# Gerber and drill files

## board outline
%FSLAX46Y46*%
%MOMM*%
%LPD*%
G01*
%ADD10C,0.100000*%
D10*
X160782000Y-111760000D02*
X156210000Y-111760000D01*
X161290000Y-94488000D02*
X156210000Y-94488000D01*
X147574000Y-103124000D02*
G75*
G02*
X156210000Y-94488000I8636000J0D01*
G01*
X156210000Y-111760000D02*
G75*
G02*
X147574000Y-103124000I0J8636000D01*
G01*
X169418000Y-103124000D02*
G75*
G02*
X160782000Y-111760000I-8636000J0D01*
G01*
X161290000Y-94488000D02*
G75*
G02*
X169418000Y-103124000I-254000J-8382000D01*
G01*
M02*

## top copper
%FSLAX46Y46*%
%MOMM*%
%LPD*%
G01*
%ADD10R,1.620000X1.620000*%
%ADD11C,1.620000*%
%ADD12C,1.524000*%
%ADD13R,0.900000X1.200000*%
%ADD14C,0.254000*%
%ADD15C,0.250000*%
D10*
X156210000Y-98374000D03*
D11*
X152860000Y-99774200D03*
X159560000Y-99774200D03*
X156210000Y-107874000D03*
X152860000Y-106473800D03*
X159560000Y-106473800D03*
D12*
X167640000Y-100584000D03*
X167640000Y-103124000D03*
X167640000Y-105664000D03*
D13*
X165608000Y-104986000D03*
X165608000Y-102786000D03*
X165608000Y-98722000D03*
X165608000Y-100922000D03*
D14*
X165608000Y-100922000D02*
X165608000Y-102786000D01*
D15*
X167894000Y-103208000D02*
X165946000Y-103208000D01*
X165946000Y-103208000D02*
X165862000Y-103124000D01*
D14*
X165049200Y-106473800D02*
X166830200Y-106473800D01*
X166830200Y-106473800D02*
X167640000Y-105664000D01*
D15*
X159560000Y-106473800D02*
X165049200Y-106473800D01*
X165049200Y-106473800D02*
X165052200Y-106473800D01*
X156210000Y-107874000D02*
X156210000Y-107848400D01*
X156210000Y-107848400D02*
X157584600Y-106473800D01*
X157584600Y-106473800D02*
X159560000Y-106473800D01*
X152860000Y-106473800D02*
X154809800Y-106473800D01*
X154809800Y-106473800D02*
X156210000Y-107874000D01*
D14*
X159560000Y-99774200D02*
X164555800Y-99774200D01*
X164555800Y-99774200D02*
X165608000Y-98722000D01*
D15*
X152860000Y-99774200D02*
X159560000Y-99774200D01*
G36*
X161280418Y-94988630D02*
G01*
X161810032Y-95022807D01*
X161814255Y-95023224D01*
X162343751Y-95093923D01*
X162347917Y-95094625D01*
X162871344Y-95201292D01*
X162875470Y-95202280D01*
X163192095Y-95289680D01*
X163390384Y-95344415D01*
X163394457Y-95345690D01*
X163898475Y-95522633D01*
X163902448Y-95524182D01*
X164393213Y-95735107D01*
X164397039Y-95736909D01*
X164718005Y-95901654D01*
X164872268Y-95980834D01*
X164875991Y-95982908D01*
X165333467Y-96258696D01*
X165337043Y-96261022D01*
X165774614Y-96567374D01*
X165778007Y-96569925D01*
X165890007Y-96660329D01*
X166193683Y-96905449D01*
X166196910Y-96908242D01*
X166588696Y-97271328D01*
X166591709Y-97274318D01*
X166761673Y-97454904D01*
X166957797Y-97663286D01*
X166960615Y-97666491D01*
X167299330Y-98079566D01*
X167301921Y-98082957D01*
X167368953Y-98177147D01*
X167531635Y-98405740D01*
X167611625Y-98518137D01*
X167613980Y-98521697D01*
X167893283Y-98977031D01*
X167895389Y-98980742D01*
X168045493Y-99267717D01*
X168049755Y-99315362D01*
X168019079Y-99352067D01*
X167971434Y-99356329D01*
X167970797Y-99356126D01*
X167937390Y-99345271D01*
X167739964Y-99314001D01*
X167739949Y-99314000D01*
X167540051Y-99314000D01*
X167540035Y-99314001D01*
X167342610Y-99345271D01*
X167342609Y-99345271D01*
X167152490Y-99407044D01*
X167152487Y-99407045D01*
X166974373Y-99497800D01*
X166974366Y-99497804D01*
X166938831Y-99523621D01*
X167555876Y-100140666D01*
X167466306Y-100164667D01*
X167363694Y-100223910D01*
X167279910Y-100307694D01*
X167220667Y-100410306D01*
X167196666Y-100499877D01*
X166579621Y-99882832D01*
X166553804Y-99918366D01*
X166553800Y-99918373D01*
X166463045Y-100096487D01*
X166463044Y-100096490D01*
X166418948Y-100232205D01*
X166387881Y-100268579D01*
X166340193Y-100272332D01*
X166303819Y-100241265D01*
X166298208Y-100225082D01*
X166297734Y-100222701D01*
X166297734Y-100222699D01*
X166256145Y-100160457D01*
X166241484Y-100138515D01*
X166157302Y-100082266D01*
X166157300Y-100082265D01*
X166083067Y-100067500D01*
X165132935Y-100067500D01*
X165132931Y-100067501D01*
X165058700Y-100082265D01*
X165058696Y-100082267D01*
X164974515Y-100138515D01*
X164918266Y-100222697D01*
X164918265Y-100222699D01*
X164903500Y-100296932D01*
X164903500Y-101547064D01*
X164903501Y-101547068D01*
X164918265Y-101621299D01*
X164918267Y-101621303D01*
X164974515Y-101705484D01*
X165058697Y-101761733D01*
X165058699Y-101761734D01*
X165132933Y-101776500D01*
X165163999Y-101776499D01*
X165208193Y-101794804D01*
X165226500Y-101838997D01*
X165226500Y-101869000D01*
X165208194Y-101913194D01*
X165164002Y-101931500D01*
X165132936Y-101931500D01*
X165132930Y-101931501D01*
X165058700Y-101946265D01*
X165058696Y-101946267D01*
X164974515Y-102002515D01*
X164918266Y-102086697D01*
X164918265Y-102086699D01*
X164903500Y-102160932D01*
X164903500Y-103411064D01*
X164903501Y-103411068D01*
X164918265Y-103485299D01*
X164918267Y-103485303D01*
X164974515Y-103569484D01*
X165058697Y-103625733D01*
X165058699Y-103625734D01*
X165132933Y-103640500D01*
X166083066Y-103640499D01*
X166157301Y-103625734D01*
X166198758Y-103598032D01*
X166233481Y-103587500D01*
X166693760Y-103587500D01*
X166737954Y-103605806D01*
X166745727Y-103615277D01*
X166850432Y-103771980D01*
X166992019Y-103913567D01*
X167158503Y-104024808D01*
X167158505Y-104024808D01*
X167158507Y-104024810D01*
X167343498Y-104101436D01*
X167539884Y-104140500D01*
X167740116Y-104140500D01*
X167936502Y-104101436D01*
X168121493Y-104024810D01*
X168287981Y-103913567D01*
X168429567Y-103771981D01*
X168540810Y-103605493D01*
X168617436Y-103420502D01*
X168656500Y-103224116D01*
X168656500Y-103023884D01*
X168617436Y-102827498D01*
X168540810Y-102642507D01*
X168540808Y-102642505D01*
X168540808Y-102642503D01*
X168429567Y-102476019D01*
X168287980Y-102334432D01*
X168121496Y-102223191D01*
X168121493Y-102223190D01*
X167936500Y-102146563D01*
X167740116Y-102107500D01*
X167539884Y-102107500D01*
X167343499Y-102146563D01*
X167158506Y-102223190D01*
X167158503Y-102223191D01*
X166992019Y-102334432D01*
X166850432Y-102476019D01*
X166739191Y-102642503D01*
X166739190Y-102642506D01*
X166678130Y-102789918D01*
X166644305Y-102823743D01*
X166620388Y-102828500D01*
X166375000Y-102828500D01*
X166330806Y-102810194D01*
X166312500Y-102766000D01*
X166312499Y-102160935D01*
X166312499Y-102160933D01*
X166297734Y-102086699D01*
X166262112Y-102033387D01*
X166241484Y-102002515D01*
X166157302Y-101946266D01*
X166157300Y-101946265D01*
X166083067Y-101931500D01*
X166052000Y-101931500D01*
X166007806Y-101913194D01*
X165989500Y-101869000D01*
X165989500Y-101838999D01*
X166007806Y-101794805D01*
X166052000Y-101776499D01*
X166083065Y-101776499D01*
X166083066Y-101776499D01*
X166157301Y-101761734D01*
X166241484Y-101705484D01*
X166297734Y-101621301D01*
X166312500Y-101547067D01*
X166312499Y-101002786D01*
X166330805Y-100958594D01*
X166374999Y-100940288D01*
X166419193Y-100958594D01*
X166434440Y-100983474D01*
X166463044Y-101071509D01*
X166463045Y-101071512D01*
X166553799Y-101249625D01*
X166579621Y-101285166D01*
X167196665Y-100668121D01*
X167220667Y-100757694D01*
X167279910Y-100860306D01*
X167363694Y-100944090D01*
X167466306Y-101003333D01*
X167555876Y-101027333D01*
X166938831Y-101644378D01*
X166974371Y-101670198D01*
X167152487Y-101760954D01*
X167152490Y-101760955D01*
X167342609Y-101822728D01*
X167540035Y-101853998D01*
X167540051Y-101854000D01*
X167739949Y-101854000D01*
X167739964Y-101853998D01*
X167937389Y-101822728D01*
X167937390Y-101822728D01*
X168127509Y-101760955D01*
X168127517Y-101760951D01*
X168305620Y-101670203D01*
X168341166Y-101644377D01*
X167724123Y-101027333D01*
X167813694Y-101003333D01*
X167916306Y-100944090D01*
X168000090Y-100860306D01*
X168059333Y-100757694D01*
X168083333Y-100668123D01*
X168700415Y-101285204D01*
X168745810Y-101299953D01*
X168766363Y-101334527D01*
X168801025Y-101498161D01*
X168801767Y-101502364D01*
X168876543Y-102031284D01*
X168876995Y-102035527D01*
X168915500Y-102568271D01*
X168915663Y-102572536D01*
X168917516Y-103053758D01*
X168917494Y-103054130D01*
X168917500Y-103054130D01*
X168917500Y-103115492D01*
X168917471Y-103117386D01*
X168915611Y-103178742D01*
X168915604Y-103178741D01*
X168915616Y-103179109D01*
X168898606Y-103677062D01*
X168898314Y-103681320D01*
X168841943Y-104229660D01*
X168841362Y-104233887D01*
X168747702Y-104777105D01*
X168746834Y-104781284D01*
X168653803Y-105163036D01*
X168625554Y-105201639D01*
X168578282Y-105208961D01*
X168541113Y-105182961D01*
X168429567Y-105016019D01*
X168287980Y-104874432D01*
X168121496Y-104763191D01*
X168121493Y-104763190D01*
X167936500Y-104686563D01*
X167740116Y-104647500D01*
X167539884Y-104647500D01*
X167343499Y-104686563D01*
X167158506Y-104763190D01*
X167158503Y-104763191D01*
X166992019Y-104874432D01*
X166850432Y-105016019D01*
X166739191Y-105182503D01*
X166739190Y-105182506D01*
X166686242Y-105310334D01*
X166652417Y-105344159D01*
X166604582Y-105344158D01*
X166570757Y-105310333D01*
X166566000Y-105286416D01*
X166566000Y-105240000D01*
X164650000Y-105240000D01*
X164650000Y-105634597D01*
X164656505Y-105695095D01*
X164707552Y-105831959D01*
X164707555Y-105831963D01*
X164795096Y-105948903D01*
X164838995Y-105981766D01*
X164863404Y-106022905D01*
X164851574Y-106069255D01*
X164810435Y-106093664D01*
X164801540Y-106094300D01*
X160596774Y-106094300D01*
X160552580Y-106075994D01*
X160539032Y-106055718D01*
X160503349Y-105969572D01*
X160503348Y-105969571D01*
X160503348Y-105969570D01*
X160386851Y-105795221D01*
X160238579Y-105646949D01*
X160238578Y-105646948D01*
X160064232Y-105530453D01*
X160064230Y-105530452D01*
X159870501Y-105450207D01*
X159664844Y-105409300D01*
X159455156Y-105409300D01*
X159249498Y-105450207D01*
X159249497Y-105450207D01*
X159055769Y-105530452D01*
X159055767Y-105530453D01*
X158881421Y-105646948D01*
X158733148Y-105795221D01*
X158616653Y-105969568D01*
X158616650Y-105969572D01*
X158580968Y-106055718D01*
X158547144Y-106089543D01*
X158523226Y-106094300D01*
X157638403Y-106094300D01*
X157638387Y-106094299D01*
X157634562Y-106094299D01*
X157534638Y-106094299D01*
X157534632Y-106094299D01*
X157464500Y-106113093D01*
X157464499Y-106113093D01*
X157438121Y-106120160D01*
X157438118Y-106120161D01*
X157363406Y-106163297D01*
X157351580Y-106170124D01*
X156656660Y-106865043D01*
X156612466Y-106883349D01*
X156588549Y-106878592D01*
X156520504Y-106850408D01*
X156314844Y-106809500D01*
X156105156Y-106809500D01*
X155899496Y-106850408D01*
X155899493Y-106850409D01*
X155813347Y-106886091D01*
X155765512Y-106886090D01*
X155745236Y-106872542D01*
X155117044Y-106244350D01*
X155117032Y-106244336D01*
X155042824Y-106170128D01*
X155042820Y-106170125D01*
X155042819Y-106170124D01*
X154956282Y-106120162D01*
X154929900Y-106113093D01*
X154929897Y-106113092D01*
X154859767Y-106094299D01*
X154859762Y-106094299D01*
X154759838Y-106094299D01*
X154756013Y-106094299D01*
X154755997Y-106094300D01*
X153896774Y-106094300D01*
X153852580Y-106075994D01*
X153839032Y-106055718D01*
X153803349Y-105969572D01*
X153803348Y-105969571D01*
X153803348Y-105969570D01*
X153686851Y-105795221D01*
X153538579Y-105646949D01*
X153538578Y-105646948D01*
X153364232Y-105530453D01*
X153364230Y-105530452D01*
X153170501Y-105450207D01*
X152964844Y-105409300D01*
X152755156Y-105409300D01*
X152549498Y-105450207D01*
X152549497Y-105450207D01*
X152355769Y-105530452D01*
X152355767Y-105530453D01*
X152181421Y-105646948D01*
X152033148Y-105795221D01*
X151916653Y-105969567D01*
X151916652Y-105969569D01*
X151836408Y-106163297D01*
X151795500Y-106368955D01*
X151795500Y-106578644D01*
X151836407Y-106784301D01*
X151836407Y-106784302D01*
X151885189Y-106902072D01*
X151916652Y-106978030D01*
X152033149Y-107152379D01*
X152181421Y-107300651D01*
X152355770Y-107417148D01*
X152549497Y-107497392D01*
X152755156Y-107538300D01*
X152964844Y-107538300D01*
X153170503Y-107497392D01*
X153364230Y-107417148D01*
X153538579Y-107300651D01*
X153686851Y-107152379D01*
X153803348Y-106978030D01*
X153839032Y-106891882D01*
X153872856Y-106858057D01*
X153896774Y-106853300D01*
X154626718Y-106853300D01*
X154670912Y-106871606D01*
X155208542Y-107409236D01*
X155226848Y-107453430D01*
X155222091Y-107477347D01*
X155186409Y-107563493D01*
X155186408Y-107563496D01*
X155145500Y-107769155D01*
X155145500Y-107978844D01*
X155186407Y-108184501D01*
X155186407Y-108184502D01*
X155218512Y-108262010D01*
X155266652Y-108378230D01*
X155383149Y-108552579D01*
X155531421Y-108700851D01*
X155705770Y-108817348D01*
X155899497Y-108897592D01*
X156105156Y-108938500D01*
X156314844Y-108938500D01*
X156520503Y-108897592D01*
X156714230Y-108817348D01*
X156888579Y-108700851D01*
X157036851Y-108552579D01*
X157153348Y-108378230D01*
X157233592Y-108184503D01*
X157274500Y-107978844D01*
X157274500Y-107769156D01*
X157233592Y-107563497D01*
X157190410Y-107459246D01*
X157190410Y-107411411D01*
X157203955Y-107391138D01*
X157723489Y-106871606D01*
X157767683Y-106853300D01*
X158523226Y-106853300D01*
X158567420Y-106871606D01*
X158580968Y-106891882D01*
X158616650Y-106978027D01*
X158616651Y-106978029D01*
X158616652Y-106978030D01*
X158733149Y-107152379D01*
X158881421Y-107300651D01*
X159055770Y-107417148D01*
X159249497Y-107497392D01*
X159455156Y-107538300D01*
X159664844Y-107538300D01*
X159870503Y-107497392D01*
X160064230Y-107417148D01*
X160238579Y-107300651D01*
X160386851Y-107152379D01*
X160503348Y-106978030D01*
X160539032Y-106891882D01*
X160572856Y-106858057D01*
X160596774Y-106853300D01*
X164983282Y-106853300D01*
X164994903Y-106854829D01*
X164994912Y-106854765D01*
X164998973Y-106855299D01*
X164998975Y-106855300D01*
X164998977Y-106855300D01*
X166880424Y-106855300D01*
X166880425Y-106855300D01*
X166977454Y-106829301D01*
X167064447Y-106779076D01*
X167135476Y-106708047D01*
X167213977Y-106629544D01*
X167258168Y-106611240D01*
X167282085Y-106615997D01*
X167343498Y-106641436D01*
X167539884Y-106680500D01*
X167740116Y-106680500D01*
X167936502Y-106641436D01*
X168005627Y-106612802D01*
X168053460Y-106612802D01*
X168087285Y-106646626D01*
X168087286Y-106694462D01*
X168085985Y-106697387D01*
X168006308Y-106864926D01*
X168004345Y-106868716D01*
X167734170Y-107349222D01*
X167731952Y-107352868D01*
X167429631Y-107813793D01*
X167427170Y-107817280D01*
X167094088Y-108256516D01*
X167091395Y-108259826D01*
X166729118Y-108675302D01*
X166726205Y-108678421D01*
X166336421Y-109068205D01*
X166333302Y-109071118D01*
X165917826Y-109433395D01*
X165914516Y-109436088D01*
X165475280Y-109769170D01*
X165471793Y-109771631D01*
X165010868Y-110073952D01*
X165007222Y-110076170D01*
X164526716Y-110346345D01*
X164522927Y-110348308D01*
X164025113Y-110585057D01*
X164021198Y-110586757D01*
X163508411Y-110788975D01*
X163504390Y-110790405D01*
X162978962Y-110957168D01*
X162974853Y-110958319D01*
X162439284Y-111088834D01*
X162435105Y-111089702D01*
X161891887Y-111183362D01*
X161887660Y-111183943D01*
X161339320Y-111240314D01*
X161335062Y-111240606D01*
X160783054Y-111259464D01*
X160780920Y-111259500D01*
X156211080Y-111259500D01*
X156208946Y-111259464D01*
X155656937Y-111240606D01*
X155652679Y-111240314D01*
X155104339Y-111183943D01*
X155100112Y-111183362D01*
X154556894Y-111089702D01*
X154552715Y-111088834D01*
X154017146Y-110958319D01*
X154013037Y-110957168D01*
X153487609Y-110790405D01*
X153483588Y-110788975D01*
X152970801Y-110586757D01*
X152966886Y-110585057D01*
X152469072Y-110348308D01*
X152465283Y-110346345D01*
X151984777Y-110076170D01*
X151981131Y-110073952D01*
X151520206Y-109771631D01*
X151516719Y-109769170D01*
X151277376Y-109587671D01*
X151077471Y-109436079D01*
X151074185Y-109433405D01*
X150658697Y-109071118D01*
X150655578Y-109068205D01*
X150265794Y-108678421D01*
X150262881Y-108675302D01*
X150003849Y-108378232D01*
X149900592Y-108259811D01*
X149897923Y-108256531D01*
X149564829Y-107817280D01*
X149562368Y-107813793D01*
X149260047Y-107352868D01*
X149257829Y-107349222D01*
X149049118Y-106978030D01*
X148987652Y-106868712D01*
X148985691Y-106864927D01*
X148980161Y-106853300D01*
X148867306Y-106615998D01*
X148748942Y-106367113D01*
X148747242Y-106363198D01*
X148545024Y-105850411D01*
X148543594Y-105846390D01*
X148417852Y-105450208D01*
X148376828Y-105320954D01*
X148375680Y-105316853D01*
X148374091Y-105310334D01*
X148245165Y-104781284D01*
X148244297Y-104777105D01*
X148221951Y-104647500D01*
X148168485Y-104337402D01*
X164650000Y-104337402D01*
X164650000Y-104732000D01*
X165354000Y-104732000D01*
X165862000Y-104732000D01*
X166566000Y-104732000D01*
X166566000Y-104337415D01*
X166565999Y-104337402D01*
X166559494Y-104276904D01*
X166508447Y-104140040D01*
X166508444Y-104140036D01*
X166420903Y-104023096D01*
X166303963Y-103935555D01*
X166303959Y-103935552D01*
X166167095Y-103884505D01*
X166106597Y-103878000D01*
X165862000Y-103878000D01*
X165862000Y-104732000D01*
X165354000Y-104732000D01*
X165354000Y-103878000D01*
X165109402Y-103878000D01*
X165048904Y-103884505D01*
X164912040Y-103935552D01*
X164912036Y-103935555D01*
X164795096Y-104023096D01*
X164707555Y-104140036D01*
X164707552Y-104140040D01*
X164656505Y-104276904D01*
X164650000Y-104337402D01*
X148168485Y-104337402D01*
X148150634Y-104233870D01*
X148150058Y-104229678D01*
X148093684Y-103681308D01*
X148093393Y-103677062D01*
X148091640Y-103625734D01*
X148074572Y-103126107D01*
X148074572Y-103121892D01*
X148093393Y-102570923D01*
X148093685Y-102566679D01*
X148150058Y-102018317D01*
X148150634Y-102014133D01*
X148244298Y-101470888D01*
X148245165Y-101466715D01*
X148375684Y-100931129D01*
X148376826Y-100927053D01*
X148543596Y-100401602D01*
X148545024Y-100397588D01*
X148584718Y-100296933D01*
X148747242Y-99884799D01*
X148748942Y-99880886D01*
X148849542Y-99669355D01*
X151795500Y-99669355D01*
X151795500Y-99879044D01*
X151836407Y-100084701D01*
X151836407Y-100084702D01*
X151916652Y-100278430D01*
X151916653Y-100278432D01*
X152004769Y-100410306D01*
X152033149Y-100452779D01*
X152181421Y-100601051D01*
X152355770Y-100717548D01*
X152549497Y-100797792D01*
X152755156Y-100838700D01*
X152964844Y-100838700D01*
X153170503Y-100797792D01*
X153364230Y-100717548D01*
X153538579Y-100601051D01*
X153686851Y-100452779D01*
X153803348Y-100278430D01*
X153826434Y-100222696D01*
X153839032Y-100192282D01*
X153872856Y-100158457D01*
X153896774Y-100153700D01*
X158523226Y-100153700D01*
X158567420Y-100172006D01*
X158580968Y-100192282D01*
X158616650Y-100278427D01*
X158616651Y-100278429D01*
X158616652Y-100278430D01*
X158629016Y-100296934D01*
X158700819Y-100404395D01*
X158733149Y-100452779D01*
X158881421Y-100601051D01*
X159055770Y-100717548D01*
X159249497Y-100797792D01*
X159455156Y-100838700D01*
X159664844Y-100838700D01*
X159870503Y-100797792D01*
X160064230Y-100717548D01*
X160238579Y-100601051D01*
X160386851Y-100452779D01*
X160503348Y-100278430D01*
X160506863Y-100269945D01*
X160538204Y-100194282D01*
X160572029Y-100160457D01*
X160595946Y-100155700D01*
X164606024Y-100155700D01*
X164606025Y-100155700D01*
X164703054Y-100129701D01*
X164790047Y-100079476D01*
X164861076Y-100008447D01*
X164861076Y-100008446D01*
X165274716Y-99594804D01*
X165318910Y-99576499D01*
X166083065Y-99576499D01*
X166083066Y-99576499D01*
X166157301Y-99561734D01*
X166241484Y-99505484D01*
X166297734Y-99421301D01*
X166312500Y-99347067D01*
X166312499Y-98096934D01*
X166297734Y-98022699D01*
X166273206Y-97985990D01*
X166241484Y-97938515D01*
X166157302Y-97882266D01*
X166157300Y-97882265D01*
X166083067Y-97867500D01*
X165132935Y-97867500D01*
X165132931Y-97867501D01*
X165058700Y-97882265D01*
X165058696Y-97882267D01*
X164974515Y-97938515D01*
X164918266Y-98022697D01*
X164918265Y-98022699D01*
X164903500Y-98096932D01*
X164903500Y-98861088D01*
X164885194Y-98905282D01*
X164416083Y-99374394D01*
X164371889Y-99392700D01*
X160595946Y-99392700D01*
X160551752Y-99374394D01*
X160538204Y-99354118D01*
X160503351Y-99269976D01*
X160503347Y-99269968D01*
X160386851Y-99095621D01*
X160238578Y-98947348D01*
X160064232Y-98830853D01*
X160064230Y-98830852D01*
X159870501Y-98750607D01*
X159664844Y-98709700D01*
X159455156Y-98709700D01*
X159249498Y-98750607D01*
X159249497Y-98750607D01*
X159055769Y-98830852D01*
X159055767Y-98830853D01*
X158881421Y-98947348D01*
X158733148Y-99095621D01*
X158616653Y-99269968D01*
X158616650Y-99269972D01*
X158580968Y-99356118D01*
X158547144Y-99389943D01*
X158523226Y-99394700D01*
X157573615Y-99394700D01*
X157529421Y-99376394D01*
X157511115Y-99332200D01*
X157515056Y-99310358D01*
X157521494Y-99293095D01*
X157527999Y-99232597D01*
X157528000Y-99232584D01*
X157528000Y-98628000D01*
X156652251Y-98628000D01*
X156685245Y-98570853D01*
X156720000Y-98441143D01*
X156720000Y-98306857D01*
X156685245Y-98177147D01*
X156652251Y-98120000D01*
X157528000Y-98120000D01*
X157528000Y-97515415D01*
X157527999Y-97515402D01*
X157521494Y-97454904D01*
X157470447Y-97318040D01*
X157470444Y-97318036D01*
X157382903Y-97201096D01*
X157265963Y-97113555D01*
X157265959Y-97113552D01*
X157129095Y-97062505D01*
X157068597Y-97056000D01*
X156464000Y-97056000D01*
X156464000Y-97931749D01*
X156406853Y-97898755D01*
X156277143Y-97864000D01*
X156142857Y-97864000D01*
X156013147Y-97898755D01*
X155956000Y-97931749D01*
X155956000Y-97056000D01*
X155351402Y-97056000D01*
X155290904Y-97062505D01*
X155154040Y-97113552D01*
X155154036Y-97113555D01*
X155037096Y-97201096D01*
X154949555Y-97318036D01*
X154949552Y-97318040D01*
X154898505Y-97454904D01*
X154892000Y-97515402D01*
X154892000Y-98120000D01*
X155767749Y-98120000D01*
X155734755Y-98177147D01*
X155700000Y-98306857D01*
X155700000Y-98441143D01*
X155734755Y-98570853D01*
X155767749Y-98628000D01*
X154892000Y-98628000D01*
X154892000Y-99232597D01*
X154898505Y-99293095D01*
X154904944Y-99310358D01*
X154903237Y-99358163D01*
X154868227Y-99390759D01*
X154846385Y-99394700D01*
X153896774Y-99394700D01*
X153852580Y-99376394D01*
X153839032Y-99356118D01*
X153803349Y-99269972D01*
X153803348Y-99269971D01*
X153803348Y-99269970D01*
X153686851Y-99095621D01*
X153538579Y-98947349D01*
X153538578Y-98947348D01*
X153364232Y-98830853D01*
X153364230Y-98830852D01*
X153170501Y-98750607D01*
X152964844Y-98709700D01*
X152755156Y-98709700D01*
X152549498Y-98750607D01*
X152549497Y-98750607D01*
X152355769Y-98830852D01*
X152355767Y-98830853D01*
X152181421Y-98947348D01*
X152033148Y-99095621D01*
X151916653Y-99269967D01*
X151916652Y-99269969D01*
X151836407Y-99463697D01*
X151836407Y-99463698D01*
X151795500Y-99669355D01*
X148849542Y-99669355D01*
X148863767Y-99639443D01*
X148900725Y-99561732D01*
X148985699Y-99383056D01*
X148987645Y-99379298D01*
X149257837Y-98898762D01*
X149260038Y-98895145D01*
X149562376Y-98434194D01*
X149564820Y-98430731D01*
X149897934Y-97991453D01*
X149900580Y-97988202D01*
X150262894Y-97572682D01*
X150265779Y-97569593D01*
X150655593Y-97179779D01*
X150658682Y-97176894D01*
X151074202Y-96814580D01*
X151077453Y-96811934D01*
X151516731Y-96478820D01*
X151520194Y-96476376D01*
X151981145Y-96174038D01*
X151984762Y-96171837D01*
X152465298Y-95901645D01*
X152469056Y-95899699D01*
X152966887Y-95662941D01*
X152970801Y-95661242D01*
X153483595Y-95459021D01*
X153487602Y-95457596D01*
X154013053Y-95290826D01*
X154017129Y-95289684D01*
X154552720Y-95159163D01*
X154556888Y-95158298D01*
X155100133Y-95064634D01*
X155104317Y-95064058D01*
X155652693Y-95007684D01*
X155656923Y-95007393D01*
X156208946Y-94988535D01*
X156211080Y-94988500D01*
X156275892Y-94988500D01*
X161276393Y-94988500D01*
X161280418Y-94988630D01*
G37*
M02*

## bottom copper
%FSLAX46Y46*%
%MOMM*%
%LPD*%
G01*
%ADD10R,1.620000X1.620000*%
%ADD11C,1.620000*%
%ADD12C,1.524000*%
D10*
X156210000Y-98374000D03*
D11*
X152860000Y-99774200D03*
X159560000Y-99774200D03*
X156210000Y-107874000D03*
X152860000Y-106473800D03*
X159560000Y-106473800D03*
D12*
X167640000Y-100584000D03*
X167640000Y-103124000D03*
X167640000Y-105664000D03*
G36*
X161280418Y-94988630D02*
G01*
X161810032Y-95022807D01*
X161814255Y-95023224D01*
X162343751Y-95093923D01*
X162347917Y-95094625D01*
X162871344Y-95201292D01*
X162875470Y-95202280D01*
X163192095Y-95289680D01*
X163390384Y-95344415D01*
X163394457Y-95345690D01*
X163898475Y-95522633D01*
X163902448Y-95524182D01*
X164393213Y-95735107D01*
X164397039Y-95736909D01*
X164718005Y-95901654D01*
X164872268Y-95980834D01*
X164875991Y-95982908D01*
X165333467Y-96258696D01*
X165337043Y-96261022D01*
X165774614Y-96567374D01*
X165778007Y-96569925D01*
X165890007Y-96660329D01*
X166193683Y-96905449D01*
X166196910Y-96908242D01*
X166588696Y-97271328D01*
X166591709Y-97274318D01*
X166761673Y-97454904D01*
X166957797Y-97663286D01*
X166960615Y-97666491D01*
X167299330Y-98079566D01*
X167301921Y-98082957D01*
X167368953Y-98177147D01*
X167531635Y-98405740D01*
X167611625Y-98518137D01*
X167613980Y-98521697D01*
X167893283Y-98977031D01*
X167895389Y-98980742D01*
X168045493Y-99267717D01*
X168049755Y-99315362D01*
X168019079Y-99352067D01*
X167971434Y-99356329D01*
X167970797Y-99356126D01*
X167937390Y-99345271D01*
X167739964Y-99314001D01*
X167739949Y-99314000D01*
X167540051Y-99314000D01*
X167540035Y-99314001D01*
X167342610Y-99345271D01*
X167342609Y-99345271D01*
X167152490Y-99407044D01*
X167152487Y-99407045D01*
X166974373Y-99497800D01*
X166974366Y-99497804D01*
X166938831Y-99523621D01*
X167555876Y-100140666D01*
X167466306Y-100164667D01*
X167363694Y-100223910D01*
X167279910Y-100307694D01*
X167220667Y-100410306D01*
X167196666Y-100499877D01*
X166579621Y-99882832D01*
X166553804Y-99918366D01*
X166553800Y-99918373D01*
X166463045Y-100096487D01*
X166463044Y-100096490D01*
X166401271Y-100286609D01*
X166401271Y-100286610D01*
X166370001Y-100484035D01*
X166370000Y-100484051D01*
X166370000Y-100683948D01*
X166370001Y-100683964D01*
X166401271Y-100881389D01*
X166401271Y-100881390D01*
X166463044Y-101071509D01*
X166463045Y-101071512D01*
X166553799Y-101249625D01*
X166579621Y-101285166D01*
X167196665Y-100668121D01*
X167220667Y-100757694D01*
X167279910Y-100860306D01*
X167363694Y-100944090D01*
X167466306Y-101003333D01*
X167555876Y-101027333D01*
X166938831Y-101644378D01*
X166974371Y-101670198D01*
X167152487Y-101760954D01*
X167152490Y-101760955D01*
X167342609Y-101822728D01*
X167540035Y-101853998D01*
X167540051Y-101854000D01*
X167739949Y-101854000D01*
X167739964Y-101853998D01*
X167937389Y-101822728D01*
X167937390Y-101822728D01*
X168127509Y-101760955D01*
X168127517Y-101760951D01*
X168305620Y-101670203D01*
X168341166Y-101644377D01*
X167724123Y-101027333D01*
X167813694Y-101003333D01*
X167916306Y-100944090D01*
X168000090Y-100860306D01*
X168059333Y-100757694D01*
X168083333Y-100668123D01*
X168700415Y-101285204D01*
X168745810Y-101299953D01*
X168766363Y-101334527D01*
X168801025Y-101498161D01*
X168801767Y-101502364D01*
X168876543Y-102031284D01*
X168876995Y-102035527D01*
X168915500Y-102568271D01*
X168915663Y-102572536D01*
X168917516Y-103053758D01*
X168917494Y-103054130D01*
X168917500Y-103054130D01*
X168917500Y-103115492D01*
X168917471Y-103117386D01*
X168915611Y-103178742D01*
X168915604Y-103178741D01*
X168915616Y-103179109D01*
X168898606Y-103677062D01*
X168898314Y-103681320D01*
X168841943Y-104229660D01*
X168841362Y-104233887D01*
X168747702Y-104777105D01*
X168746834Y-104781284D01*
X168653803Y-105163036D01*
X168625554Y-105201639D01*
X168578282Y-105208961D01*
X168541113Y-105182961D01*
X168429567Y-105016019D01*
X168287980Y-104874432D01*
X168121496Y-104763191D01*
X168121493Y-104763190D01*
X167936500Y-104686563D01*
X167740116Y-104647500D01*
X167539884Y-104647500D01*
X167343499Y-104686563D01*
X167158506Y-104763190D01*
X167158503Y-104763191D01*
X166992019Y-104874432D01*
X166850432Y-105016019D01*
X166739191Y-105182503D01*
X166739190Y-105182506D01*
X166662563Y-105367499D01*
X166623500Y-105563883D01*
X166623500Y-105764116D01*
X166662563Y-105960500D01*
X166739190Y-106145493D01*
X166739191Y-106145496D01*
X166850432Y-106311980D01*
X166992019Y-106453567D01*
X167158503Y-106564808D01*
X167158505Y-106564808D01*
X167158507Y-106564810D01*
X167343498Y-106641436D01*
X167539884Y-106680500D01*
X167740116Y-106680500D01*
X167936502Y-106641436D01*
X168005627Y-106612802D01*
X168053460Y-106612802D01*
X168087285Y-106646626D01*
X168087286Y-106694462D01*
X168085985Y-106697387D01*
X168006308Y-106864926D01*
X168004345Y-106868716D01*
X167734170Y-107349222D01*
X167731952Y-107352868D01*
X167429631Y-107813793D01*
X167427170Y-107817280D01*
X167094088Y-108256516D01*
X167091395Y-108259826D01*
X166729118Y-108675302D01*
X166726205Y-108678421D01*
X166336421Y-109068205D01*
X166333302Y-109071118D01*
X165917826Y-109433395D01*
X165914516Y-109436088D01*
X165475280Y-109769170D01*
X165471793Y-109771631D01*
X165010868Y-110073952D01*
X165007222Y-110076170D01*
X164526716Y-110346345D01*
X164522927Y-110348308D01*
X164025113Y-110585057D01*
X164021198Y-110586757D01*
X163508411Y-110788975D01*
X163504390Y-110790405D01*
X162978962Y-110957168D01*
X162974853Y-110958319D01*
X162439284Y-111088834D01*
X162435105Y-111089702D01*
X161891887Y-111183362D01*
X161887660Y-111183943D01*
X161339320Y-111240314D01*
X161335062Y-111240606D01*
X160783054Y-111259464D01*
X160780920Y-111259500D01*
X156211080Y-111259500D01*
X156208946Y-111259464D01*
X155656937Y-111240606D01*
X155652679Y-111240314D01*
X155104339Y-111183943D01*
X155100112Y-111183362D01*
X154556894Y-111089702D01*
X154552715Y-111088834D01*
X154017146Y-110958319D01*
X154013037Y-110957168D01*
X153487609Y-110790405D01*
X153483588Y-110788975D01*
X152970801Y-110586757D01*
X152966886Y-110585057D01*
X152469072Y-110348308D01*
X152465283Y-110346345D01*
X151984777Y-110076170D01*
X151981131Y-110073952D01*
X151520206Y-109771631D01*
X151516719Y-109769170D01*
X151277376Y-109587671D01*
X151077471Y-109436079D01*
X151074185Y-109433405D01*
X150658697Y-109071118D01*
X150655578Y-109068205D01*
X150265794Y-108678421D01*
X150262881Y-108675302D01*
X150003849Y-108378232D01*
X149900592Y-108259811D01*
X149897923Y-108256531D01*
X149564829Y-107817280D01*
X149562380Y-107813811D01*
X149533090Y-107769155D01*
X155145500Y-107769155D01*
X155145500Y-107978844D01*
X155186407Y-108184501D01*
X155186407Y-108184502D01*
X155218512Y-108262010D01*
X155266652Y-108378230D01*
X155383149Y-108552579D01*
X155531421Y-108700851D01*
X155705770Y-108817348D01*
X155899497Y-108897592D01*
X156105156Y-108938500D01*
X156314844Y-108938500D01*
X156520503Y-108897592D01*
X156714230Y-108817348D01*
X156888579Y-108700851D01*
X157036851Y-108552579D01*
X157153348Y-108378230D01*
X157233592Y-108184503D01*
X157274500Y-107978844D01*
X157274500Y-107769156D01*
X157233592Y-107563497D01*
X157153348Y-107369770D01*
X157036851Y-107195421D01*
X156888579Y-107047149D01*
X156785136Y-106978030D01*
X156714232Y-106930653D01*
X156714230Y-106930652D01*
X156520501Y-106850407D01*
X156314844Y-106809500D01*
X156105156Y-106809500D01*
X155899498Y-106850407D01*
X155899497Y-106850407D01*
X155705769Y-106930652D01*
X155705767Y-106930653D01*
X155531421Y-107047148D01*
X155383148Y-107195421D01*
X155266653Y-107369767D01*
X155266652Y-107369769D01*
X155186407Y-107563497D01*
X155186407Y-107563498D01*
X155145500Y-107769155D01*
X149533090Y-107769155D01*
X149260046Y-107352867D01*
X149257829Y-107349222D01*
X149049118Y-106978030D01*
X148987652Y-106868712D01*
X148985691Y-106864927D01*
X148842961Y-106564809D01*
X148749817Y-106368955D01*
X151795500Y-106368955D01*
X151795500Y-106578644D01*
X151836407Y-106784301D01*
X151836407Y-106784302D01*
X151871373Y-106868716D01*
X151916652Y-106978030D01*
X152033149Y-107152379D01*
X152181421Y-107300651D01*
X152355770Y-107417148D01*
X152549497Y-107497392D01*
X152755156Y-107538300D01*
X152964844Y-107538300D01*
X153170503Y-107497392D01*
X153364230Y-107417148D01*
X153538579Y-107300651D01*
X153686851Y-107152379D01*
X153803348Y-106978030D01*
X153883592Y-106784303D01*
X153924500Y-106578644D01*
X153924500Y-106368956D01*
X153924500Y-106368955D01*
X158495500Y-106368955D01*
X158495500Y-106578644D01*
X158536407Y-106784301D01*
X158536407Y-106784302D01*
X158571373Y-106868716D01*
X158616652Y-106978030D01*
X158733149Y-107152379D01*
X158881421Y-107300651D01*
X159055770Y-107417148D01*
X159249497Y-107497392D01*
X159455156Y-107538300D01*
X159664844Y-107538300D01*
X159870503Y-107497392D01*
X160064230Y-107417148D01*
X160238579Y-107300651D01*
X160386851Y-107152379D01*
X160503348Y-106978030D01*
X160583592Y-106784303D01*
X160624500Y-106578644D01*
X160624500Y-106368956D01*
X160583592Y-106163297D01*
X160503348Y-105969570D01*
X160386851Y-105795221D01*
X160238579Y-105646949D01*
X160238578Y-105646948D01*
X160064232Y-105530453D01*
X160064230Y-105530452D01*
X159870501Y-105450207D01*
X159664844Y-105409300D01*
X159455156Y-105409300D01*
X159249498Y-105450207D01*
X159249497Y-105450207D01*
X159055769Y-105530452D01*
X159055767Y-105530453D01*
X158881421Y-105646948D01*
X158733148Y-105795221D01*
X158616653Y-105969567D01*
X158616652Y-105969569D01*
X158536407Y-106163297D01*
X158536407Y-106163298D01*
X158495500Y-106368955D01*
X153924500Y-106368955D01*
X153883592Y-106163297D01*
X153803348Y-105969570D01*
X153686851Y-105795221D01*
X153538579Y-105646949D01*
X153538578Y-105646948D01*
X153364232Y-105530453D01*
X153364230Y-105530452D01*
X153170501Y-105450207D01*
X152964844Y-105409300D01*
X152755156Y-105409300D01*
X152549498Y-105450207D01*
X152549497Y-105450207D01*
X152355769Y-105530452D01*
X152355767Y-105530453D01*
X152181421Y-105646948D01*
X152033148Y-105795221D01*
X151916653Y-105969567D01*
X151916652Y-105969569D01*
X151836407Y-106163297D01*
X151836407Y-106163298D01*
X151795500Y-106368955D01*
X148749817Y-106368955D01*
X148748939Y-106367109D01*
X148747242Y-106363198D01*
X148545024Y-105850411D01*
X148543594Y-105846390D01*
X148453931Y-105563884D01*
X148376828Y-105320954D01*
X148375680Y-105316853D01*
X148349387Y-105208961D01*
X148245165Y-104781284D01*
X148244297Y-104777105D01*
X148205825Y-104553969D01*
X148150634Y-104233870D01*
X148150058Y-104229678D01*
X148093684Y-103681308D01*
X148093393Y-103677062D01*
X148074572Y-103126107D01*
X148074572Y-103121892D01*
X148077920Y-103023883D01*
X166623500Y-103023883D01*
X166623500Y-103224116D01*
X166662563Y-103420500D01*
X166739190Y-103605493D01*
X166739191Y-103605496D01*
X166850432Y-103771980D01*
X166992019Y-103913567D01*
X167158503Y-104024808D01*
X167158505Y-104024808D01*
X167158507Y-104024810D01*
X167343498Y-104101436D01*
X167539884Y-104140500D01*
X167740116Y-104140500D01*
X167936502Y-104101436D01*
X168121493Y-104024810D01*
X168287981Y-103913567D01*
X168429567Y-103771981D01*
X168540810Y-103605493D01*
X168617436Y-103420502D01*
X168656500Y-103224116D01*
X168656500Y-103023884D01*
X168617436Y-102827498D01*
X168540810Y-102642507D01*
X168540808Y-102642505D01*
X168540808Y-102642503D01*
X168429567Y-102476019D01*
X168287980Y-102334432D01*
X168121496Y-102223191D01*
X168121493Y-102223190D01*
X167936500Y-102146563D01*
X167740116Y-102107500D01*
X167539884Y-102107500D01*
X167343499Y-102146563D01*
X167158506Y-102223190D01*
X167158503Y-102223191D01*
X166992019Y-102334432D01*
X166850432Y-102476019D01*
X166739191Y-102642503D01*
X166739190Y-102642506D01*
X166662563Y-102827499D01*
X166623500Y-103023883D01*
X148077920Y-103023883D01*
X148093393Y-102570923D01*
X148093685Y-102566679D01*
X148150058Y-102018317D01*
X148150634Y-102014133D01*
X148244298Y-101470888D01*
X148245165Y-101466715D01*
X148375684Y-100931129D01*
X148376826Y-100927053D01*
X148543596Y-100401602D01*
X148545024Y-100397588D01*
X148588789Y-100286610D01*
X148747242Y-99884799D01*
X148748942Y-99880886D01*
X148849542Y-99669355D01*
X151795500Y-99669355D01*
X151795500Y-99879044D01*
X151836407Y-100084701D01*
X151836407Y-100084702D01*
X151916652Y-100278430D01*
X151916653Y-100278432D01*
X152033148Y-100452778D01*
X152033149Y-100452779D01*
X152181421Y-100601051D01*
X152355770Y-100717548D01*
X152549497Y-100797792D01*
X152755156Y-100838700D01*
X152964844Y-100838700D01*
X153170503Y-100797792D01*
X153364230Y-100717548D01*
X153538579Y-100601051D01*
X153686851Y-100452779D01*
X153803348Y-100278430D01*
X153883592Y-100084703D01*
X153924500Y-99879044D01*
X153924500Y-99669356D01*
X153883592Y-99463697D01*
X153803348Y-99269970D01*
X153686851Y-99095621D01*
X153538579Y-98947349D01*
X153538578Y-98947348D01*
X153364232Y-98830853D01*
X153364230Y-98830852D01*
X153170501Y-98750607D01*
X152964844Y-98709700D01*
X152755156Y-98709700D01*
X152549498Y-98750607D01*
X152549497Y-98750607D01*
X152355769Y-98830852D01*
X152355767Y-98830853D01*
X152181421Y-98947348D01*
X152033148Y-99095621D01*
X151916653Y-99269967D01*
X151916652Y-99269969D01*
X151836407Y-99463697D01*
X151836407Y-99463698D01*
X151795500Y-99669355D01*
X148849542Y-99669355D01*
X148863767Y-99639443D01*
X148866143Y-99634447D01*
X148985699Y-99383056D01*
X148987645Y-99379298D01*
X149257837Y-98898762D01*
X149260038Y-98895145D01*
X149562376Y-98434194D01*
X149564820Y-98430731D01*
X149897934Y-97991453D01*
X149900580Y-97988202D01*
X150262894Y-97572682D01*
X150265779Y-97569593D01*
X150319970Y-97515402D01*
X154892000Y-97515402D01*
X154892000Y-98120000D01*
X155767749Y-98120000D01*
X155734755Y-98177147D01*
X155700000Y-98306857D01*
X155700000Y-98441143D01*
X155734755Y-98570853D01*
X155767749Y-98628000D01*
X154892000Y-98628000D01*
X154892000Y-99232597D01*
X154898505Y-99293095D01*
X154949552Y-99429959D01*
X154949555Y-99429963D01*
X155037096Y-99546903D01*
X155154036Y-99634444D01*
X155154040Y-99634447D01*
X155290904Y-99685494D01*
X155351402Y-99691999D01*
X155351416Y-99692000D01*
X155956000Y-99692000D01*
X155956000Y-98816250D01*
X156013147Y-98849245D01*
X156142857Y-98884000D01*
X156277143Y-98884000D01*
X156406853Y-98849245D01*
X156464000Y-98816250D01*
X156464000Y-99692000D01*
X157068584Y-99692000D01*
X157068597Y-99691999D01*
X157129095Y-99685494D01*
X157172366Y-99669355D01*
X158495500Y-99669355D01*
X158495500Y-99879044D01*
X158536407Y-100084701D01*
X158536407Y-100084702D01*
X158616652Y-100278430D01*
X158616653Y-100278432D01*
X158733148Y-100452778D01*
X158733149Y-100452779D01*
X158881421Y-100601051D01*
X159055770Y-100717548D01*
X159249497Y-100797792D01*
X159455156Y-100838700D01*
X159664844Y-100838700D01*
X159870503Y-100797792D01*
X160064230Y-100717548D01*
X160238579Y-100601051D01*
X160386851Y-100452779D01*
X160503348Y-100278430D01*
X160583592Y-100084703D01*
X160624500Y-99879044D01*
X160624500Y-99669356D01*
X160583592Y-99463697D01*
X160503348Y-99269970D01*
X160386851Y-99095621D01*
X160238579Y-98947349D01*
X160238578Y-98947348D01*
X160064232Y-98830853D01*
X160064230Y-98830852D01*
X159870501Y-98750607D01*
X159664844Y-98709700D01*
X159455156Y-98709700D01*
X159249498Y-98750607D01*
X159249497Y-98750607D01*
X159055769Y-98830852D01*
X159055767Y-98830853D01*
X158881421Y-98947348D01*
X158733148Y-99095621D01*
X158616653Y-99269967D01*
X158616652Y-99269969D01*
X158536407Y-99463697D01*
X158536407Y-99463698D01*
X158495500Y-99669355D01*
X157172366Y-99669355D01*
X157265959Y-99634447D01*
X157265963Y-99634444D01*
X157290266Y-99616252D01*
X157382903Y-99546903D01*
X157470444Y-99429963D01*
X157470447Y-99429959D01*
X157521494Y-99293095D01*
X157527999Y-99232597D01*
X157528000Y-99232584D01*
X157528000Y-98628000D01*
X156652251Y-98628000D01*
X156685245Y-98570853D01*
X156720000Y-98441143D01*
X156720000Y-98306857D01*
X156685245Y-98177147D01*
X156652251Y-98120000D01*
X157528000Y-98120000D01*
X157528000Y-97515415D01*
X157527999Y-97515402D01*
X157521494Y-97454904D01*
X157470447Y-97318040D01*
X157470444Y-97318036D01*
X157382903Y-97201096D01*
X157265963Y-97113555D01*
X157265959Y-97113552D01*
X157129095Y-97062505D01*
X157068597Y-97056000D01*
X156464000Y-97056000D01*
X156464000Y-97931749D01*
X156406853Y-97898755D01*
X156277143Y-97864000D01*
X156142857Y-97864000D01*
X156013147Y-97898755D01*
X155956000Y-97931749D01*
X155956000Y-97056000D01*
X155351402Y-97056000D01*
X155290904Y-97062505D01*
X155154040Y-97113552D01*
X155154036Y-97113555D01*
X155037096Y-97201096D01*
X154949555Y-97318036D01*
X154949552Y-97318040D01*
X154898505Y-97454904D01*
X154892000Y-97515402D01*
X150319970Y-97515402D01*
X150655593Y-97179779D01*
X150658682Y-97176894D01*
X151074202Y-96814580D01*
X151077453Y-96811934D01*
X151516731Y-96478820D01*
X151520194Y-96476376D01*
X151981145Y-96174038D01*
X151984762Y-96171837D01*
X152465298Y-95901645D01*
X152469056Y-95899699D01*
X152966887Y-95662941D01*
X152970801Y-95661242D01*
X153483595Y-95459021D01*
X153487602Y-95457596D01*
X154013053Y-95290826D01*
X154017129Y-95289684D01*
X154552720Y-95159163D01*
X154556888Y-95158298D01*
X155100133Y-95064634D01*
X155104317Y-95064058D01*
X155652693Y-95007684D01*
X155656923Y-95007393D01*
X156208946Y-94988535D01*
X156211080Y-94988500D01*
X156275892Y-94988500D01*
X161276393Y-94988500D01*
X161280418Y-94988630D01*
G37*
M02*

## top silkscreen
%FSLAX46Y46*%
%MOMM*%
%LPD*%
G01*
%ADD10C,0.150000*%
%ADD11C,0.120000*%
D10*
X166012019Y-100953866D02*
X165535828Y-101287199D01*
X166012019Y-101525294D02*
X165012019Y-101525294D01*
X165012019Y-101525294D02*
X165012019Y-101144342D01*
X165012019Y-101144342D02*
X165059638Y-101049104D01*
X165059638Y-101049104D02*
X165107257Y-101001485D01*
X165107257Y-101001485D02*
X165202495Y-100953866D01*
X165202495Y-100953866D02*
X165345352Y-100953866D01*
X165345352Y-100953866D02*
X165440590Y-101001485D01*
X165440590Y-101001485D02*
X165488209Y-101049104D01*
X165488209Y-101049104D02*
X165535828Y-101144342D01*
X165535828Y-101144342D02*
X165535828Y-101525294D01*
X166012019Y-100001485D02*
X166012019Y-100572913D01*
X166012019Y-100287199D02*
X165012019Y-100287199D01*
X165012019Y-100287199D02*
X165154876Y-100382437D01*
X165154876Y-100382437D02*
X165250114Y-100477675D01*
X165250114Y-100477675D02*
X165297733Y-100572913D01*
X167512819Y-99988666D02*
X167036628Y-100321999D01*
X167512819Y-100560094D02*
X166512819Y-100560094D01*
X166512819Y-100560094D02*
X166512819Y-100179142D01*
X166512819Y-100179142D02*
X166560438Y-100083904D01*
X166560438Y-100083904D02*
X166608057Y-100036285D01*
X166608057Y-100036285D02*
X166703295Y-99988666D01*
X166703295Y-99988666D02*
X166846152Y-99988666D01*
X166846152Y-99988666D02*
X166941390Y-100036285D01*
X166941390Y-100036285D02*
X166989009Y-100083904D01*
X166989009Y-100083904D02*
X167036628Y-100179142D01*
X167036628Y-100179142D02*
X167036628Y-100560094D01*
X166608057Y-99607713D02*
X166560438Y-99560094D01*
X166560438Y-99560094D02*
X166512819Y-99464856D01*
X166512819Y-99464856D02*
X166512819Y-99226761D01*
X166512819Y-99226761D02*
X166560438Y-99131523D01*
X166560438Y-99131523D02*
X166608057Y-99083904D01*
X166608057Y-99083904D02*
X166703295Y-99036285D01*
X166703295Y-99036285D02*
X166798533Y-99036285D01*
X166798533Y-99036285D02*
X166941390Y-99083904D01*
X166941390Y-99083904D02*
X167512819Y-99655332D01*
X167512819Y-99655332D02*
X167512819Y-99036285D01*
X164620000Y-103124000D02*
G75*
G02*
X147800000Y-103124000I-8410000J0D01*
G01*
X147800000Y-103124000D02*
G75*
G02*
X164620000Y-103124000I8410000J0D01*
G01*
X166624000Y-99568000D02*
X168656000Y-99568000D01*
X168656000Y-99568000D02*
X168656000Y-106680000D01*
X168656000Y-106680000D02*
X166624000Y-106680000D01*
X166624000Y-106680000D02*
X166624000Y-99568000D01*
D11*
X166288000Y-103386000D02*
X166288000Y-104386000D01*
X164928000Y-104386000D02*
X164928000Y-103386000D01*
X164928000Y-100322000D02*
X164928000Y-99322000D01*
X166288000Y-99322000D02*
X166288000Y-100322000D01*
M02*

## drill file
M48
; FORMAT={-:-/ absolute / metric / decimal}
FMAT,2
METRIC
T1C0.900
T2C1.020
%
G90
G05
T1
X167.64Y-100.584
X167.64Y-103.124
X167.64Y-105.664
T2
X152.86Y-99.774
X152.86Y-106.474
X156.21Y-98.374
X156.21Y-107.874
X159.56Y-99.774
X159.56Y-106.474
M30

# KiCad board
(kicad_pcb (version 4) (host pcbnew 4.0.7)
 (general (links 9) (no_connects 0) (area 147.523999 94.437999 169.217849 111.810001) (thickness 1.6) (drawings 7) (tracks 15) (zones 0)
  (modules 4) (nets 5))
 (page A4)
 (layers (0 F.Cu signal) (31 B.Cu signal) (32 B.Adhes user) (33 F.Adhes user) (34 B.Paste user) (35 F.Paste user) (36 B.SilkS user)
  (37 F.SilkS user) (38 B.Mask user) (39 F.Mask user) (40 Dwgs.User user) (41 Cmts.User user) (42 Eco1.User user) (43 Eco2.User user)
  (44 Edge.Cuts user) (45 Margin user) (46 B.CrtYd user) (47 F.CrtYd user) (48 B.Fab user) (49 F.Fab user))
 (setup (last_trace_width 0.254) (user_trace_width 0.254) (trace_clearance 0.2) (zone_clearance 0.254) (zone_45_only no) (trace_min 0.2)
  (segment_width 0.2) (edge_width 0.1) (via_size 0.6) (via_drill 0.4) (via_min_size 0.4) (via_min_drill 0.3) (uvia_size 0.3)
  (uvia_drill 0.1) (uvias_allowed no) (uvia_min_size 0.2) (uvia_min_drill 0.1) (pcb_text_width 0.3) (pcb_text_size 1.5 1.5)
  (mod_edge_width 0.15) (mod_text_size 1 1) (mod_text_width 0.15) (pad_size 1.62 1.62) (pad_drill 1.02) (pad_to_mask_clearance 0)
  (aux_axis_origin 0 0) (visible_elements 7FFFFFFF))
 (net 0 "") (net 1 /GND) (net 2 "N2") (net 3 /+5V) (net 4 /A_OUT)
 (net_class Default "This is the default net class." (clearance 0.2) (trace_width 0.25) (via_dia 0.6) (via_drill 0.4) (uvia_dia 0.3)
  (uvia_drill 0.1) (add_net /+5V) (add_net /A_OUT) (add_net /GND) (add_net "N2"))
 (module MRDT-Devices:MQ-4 (layer F.Cu) (at 156.21 103.124 90)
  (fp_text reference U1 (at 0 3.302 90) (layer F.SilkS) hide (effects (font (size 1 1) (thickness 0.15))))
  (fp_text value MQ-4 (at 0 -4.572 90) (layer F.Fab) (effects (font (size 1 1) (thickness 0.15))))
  (fp_circle (center 0 0) (end 8.41 0) (layer F.SilkS) (width 0.15))
  (pad 3 thru_hole rect (at 4.75 0 90) (size 1.62 1.62) (drill 1.02) (layers *.Cu *.Mask) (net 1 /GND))
  (pad 2 thru_hole circle (at 3.3498 -3.35 90) (size 1.62 1.62) (drill 1.02) (layers *.Cu *.Mask) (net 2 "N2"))
  (pad 2 thru_hole circle (at 3.3498 3.35 90) (size 1.62 1.62) (drill 1.02) (layers *.Cu *.Mask) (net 2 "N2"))
  (pad 1 thru_hole circle (at -4.75 0 90) (size 1.62 1.62) (drill 1.02) (layers *.Cu *.Mask) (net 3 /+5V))
  (pad 1 thru_hole circle (at -3.3498 -3.35 90) (size 1.62 1.62) (drill 1.02) (layers *.Cu *.Mask) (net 3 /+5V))
  (pad 1 thru_hole circle (at -3.3498 3.35 90) (size 1.62 1.62) (drill 1.02) (layers *.Cu *.Mask) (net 3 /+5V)))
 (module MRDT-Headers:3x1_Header (layer F.Cu) (at 167.132 104.14)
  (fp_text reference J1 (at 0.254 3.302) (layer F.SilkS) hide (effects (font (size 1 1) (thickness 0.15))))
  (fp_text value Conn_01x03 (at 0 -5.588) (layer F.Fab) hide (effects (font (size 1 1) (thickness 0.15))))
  (fp_line (start -0.508 -4.572) (end 1.524 -4.572) (layer F.SilkS) (width 0.15))
  (fp_line (start 1.524 -4.572) (end 1.524 2.54) (layer F.SilkS) (width 0.15))
  (fp_line (start 1.524 2.54) (end -0.508 2.54) (layer F.SilkS) (width 0.15))
  (fp_line (start -0.508 2.54) (end -0.508 -4.572) (layer F.SilkS) (width 0.15))
  (pad 1 thru_hole circle (at 0.508 -3.556) (size 1.524 1.524) (drill 0.9) (layers *.Cu *.Mask) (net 1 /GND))
  (pad 2 thru_hole circle (at 0.508 -1.016) (size 1.524 1.524) (drill 0.9) (layers *.Cu *.Mask) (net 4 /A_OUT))
  (pad 3 thru_hole circle (at 0.508 1.524) (size 1.524 1.524) (drill 0.9) (layers *.Cu *.Mask) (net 3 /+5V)))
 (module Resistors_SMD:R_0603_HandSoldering (layer F.Cu) (at 165.608 103.886 90)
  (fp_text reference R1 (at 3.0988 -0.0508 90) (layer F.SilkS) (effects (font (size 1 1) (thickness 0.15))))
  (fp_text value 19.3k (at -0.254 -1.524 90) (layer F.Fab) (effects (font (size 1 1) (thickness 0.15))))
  (fp_line (start 0.5 0.68) (end -0.5 0.68) (layer F.SilkS) (width 0.12))
  (fp_line (start -0.5 -0.68) (end 0.5 -0.68) (layer F.SilkS) (width 0.12))
  (pad 1 smd rect (at -1.1 0 90) (size 1.2 0.9) (layers F.Cu F.Paste F.Mask) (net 1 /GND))
  (pad 2 smd rect (at 1.1 0 90) (size 1.2 0.9) (layers F.Cu F.Paste F.Mask) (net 4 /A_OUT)))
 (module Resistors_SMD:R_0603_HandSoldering (layer F.Cu) (at 165.608 99.822 270)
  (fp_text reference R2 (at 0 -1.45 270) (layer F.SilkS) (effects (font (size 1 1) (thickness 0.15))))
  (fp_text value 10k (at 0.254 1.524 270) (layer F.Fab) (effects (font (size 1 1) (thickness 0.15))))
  (fp_line (start 0.5 0.68) (end -0.5 0.68) (layer F.SilkS) (width 0.12))
  (fp_line (start -0.5 -0.68) (end 0.5 -0.68) (layer F.SilkS) (width 0.12))
  (pad 1 smd rect (at -1.1 0 270) (size 1.2 0.9) (layers F.Cu F.Paste F.Mask) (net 2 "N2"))
  (pad 2 smd rect (at 1.1 0 270) (size 1.2 0.9) (layers F.Cu F.Paste F.Mask) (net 4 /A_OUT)))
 (gr_line (start 160.782 111.76) (end 156.21 111.76) (angle 90) (layer Edge.Cuts) (width 0.1))
 (gr_line (start 161.29 94.488) (end 156.21 94.488) (angle 90) (layer Edge.Cuts) (width 0.1))
 (gr_arc (start 156.21 103.124) (end 147.574 103.124) (angle 90) (layer Edge.Cuts) (width 0.1))
 (gr_arc (start 156.21 103.124) (end 156.21 111.76) (angle 90) (layer Edge.Cuts) (width 0.1))
 (gr_arc (start 160.782 103.124) (end 169.418 103.124) (angle 90) (layer Edge.Cuts) (width 0.1))
 (gr_arc (start 161.036 102.87) (end 161.29 94.488) (angle 90) (layer Edge.Cuts) (width 0.1))
 (segment (start 165.608 100.922) (end 165.608 102.786) (width 0.254) (layer F.Cu) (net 4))
 (segment (start 167.894 103.208) (end 165.946 103.208) (width 0.25) (layer F.Cu) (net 4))
 (segment (start 165.946 103.208) (end 165.862 103.124) (width 0.25) (layer F.Cu) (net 4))
 (segment (start 165.0492 106.4738) (end 166.8302 106.4738) (width 0.254) (layer F.Cu) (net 3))
 (segment (start 166.8302 106.4738) (end 167.64 105.664) (width 0.254) (layer F.Cu) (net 3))
 (segment (start 159.56 106.4738) (end 165.0492 106.4738) (width 0.25) (layer F.Cu) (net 3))
 (segment (start 165.0492 106.4738) (end 165.0522 106.4738) (width 0.25) (layer F.Cu) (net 3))
 (segment (start 156.21 107.874) (end 156.21 107.8484) (width 0.25) (layer F.Cu) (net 3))
 (segment (start 156.21 107.8484) (end 157.5846 106.4738) (width 0.25) (layer F.Cu) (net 3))
 (segment (start 157.5846 106.4738) (end 159.56 106.4738) (width 0.25) (layer F.Cu) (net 3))
 (segment (start 152.86 106.4738) (end 154.8098 106.4738) (width 0.25) (layer F.Cu) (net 3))
 (segment (start 154.8098 106.4738) (end 156.21 107.874) (width 0.25) (layer F.Cu) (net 3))
 (segment (start 159.56 99.7742) (end 164.5558 99.7742) (width 0.254) (layer F.Cu) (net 2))
 (segment (start 164.5558 99.7742) (end 165.608 98.722) (width 0.254) (layer F.Cu) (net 2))
 (segment (start 152.86 99.7742) (end 159.56 99.7742) (width 0.25) (layer F.Cu) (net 2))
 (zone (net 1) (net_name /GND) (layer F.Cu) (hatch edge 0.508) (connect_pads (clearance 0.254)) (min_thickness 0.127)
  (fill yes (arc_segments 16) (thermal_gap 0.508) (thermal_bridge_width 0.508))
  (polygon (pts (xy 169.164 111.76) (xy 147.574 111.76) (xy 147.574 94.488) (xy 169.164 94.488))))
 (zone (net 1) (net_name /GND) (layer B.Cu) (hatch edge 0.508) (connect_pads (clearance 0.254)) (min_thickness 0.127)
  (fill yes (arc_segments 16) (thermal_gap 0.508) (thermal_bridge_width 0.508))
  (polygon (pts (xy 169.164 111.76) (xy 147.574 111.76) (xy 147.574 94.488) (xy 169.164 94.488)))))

